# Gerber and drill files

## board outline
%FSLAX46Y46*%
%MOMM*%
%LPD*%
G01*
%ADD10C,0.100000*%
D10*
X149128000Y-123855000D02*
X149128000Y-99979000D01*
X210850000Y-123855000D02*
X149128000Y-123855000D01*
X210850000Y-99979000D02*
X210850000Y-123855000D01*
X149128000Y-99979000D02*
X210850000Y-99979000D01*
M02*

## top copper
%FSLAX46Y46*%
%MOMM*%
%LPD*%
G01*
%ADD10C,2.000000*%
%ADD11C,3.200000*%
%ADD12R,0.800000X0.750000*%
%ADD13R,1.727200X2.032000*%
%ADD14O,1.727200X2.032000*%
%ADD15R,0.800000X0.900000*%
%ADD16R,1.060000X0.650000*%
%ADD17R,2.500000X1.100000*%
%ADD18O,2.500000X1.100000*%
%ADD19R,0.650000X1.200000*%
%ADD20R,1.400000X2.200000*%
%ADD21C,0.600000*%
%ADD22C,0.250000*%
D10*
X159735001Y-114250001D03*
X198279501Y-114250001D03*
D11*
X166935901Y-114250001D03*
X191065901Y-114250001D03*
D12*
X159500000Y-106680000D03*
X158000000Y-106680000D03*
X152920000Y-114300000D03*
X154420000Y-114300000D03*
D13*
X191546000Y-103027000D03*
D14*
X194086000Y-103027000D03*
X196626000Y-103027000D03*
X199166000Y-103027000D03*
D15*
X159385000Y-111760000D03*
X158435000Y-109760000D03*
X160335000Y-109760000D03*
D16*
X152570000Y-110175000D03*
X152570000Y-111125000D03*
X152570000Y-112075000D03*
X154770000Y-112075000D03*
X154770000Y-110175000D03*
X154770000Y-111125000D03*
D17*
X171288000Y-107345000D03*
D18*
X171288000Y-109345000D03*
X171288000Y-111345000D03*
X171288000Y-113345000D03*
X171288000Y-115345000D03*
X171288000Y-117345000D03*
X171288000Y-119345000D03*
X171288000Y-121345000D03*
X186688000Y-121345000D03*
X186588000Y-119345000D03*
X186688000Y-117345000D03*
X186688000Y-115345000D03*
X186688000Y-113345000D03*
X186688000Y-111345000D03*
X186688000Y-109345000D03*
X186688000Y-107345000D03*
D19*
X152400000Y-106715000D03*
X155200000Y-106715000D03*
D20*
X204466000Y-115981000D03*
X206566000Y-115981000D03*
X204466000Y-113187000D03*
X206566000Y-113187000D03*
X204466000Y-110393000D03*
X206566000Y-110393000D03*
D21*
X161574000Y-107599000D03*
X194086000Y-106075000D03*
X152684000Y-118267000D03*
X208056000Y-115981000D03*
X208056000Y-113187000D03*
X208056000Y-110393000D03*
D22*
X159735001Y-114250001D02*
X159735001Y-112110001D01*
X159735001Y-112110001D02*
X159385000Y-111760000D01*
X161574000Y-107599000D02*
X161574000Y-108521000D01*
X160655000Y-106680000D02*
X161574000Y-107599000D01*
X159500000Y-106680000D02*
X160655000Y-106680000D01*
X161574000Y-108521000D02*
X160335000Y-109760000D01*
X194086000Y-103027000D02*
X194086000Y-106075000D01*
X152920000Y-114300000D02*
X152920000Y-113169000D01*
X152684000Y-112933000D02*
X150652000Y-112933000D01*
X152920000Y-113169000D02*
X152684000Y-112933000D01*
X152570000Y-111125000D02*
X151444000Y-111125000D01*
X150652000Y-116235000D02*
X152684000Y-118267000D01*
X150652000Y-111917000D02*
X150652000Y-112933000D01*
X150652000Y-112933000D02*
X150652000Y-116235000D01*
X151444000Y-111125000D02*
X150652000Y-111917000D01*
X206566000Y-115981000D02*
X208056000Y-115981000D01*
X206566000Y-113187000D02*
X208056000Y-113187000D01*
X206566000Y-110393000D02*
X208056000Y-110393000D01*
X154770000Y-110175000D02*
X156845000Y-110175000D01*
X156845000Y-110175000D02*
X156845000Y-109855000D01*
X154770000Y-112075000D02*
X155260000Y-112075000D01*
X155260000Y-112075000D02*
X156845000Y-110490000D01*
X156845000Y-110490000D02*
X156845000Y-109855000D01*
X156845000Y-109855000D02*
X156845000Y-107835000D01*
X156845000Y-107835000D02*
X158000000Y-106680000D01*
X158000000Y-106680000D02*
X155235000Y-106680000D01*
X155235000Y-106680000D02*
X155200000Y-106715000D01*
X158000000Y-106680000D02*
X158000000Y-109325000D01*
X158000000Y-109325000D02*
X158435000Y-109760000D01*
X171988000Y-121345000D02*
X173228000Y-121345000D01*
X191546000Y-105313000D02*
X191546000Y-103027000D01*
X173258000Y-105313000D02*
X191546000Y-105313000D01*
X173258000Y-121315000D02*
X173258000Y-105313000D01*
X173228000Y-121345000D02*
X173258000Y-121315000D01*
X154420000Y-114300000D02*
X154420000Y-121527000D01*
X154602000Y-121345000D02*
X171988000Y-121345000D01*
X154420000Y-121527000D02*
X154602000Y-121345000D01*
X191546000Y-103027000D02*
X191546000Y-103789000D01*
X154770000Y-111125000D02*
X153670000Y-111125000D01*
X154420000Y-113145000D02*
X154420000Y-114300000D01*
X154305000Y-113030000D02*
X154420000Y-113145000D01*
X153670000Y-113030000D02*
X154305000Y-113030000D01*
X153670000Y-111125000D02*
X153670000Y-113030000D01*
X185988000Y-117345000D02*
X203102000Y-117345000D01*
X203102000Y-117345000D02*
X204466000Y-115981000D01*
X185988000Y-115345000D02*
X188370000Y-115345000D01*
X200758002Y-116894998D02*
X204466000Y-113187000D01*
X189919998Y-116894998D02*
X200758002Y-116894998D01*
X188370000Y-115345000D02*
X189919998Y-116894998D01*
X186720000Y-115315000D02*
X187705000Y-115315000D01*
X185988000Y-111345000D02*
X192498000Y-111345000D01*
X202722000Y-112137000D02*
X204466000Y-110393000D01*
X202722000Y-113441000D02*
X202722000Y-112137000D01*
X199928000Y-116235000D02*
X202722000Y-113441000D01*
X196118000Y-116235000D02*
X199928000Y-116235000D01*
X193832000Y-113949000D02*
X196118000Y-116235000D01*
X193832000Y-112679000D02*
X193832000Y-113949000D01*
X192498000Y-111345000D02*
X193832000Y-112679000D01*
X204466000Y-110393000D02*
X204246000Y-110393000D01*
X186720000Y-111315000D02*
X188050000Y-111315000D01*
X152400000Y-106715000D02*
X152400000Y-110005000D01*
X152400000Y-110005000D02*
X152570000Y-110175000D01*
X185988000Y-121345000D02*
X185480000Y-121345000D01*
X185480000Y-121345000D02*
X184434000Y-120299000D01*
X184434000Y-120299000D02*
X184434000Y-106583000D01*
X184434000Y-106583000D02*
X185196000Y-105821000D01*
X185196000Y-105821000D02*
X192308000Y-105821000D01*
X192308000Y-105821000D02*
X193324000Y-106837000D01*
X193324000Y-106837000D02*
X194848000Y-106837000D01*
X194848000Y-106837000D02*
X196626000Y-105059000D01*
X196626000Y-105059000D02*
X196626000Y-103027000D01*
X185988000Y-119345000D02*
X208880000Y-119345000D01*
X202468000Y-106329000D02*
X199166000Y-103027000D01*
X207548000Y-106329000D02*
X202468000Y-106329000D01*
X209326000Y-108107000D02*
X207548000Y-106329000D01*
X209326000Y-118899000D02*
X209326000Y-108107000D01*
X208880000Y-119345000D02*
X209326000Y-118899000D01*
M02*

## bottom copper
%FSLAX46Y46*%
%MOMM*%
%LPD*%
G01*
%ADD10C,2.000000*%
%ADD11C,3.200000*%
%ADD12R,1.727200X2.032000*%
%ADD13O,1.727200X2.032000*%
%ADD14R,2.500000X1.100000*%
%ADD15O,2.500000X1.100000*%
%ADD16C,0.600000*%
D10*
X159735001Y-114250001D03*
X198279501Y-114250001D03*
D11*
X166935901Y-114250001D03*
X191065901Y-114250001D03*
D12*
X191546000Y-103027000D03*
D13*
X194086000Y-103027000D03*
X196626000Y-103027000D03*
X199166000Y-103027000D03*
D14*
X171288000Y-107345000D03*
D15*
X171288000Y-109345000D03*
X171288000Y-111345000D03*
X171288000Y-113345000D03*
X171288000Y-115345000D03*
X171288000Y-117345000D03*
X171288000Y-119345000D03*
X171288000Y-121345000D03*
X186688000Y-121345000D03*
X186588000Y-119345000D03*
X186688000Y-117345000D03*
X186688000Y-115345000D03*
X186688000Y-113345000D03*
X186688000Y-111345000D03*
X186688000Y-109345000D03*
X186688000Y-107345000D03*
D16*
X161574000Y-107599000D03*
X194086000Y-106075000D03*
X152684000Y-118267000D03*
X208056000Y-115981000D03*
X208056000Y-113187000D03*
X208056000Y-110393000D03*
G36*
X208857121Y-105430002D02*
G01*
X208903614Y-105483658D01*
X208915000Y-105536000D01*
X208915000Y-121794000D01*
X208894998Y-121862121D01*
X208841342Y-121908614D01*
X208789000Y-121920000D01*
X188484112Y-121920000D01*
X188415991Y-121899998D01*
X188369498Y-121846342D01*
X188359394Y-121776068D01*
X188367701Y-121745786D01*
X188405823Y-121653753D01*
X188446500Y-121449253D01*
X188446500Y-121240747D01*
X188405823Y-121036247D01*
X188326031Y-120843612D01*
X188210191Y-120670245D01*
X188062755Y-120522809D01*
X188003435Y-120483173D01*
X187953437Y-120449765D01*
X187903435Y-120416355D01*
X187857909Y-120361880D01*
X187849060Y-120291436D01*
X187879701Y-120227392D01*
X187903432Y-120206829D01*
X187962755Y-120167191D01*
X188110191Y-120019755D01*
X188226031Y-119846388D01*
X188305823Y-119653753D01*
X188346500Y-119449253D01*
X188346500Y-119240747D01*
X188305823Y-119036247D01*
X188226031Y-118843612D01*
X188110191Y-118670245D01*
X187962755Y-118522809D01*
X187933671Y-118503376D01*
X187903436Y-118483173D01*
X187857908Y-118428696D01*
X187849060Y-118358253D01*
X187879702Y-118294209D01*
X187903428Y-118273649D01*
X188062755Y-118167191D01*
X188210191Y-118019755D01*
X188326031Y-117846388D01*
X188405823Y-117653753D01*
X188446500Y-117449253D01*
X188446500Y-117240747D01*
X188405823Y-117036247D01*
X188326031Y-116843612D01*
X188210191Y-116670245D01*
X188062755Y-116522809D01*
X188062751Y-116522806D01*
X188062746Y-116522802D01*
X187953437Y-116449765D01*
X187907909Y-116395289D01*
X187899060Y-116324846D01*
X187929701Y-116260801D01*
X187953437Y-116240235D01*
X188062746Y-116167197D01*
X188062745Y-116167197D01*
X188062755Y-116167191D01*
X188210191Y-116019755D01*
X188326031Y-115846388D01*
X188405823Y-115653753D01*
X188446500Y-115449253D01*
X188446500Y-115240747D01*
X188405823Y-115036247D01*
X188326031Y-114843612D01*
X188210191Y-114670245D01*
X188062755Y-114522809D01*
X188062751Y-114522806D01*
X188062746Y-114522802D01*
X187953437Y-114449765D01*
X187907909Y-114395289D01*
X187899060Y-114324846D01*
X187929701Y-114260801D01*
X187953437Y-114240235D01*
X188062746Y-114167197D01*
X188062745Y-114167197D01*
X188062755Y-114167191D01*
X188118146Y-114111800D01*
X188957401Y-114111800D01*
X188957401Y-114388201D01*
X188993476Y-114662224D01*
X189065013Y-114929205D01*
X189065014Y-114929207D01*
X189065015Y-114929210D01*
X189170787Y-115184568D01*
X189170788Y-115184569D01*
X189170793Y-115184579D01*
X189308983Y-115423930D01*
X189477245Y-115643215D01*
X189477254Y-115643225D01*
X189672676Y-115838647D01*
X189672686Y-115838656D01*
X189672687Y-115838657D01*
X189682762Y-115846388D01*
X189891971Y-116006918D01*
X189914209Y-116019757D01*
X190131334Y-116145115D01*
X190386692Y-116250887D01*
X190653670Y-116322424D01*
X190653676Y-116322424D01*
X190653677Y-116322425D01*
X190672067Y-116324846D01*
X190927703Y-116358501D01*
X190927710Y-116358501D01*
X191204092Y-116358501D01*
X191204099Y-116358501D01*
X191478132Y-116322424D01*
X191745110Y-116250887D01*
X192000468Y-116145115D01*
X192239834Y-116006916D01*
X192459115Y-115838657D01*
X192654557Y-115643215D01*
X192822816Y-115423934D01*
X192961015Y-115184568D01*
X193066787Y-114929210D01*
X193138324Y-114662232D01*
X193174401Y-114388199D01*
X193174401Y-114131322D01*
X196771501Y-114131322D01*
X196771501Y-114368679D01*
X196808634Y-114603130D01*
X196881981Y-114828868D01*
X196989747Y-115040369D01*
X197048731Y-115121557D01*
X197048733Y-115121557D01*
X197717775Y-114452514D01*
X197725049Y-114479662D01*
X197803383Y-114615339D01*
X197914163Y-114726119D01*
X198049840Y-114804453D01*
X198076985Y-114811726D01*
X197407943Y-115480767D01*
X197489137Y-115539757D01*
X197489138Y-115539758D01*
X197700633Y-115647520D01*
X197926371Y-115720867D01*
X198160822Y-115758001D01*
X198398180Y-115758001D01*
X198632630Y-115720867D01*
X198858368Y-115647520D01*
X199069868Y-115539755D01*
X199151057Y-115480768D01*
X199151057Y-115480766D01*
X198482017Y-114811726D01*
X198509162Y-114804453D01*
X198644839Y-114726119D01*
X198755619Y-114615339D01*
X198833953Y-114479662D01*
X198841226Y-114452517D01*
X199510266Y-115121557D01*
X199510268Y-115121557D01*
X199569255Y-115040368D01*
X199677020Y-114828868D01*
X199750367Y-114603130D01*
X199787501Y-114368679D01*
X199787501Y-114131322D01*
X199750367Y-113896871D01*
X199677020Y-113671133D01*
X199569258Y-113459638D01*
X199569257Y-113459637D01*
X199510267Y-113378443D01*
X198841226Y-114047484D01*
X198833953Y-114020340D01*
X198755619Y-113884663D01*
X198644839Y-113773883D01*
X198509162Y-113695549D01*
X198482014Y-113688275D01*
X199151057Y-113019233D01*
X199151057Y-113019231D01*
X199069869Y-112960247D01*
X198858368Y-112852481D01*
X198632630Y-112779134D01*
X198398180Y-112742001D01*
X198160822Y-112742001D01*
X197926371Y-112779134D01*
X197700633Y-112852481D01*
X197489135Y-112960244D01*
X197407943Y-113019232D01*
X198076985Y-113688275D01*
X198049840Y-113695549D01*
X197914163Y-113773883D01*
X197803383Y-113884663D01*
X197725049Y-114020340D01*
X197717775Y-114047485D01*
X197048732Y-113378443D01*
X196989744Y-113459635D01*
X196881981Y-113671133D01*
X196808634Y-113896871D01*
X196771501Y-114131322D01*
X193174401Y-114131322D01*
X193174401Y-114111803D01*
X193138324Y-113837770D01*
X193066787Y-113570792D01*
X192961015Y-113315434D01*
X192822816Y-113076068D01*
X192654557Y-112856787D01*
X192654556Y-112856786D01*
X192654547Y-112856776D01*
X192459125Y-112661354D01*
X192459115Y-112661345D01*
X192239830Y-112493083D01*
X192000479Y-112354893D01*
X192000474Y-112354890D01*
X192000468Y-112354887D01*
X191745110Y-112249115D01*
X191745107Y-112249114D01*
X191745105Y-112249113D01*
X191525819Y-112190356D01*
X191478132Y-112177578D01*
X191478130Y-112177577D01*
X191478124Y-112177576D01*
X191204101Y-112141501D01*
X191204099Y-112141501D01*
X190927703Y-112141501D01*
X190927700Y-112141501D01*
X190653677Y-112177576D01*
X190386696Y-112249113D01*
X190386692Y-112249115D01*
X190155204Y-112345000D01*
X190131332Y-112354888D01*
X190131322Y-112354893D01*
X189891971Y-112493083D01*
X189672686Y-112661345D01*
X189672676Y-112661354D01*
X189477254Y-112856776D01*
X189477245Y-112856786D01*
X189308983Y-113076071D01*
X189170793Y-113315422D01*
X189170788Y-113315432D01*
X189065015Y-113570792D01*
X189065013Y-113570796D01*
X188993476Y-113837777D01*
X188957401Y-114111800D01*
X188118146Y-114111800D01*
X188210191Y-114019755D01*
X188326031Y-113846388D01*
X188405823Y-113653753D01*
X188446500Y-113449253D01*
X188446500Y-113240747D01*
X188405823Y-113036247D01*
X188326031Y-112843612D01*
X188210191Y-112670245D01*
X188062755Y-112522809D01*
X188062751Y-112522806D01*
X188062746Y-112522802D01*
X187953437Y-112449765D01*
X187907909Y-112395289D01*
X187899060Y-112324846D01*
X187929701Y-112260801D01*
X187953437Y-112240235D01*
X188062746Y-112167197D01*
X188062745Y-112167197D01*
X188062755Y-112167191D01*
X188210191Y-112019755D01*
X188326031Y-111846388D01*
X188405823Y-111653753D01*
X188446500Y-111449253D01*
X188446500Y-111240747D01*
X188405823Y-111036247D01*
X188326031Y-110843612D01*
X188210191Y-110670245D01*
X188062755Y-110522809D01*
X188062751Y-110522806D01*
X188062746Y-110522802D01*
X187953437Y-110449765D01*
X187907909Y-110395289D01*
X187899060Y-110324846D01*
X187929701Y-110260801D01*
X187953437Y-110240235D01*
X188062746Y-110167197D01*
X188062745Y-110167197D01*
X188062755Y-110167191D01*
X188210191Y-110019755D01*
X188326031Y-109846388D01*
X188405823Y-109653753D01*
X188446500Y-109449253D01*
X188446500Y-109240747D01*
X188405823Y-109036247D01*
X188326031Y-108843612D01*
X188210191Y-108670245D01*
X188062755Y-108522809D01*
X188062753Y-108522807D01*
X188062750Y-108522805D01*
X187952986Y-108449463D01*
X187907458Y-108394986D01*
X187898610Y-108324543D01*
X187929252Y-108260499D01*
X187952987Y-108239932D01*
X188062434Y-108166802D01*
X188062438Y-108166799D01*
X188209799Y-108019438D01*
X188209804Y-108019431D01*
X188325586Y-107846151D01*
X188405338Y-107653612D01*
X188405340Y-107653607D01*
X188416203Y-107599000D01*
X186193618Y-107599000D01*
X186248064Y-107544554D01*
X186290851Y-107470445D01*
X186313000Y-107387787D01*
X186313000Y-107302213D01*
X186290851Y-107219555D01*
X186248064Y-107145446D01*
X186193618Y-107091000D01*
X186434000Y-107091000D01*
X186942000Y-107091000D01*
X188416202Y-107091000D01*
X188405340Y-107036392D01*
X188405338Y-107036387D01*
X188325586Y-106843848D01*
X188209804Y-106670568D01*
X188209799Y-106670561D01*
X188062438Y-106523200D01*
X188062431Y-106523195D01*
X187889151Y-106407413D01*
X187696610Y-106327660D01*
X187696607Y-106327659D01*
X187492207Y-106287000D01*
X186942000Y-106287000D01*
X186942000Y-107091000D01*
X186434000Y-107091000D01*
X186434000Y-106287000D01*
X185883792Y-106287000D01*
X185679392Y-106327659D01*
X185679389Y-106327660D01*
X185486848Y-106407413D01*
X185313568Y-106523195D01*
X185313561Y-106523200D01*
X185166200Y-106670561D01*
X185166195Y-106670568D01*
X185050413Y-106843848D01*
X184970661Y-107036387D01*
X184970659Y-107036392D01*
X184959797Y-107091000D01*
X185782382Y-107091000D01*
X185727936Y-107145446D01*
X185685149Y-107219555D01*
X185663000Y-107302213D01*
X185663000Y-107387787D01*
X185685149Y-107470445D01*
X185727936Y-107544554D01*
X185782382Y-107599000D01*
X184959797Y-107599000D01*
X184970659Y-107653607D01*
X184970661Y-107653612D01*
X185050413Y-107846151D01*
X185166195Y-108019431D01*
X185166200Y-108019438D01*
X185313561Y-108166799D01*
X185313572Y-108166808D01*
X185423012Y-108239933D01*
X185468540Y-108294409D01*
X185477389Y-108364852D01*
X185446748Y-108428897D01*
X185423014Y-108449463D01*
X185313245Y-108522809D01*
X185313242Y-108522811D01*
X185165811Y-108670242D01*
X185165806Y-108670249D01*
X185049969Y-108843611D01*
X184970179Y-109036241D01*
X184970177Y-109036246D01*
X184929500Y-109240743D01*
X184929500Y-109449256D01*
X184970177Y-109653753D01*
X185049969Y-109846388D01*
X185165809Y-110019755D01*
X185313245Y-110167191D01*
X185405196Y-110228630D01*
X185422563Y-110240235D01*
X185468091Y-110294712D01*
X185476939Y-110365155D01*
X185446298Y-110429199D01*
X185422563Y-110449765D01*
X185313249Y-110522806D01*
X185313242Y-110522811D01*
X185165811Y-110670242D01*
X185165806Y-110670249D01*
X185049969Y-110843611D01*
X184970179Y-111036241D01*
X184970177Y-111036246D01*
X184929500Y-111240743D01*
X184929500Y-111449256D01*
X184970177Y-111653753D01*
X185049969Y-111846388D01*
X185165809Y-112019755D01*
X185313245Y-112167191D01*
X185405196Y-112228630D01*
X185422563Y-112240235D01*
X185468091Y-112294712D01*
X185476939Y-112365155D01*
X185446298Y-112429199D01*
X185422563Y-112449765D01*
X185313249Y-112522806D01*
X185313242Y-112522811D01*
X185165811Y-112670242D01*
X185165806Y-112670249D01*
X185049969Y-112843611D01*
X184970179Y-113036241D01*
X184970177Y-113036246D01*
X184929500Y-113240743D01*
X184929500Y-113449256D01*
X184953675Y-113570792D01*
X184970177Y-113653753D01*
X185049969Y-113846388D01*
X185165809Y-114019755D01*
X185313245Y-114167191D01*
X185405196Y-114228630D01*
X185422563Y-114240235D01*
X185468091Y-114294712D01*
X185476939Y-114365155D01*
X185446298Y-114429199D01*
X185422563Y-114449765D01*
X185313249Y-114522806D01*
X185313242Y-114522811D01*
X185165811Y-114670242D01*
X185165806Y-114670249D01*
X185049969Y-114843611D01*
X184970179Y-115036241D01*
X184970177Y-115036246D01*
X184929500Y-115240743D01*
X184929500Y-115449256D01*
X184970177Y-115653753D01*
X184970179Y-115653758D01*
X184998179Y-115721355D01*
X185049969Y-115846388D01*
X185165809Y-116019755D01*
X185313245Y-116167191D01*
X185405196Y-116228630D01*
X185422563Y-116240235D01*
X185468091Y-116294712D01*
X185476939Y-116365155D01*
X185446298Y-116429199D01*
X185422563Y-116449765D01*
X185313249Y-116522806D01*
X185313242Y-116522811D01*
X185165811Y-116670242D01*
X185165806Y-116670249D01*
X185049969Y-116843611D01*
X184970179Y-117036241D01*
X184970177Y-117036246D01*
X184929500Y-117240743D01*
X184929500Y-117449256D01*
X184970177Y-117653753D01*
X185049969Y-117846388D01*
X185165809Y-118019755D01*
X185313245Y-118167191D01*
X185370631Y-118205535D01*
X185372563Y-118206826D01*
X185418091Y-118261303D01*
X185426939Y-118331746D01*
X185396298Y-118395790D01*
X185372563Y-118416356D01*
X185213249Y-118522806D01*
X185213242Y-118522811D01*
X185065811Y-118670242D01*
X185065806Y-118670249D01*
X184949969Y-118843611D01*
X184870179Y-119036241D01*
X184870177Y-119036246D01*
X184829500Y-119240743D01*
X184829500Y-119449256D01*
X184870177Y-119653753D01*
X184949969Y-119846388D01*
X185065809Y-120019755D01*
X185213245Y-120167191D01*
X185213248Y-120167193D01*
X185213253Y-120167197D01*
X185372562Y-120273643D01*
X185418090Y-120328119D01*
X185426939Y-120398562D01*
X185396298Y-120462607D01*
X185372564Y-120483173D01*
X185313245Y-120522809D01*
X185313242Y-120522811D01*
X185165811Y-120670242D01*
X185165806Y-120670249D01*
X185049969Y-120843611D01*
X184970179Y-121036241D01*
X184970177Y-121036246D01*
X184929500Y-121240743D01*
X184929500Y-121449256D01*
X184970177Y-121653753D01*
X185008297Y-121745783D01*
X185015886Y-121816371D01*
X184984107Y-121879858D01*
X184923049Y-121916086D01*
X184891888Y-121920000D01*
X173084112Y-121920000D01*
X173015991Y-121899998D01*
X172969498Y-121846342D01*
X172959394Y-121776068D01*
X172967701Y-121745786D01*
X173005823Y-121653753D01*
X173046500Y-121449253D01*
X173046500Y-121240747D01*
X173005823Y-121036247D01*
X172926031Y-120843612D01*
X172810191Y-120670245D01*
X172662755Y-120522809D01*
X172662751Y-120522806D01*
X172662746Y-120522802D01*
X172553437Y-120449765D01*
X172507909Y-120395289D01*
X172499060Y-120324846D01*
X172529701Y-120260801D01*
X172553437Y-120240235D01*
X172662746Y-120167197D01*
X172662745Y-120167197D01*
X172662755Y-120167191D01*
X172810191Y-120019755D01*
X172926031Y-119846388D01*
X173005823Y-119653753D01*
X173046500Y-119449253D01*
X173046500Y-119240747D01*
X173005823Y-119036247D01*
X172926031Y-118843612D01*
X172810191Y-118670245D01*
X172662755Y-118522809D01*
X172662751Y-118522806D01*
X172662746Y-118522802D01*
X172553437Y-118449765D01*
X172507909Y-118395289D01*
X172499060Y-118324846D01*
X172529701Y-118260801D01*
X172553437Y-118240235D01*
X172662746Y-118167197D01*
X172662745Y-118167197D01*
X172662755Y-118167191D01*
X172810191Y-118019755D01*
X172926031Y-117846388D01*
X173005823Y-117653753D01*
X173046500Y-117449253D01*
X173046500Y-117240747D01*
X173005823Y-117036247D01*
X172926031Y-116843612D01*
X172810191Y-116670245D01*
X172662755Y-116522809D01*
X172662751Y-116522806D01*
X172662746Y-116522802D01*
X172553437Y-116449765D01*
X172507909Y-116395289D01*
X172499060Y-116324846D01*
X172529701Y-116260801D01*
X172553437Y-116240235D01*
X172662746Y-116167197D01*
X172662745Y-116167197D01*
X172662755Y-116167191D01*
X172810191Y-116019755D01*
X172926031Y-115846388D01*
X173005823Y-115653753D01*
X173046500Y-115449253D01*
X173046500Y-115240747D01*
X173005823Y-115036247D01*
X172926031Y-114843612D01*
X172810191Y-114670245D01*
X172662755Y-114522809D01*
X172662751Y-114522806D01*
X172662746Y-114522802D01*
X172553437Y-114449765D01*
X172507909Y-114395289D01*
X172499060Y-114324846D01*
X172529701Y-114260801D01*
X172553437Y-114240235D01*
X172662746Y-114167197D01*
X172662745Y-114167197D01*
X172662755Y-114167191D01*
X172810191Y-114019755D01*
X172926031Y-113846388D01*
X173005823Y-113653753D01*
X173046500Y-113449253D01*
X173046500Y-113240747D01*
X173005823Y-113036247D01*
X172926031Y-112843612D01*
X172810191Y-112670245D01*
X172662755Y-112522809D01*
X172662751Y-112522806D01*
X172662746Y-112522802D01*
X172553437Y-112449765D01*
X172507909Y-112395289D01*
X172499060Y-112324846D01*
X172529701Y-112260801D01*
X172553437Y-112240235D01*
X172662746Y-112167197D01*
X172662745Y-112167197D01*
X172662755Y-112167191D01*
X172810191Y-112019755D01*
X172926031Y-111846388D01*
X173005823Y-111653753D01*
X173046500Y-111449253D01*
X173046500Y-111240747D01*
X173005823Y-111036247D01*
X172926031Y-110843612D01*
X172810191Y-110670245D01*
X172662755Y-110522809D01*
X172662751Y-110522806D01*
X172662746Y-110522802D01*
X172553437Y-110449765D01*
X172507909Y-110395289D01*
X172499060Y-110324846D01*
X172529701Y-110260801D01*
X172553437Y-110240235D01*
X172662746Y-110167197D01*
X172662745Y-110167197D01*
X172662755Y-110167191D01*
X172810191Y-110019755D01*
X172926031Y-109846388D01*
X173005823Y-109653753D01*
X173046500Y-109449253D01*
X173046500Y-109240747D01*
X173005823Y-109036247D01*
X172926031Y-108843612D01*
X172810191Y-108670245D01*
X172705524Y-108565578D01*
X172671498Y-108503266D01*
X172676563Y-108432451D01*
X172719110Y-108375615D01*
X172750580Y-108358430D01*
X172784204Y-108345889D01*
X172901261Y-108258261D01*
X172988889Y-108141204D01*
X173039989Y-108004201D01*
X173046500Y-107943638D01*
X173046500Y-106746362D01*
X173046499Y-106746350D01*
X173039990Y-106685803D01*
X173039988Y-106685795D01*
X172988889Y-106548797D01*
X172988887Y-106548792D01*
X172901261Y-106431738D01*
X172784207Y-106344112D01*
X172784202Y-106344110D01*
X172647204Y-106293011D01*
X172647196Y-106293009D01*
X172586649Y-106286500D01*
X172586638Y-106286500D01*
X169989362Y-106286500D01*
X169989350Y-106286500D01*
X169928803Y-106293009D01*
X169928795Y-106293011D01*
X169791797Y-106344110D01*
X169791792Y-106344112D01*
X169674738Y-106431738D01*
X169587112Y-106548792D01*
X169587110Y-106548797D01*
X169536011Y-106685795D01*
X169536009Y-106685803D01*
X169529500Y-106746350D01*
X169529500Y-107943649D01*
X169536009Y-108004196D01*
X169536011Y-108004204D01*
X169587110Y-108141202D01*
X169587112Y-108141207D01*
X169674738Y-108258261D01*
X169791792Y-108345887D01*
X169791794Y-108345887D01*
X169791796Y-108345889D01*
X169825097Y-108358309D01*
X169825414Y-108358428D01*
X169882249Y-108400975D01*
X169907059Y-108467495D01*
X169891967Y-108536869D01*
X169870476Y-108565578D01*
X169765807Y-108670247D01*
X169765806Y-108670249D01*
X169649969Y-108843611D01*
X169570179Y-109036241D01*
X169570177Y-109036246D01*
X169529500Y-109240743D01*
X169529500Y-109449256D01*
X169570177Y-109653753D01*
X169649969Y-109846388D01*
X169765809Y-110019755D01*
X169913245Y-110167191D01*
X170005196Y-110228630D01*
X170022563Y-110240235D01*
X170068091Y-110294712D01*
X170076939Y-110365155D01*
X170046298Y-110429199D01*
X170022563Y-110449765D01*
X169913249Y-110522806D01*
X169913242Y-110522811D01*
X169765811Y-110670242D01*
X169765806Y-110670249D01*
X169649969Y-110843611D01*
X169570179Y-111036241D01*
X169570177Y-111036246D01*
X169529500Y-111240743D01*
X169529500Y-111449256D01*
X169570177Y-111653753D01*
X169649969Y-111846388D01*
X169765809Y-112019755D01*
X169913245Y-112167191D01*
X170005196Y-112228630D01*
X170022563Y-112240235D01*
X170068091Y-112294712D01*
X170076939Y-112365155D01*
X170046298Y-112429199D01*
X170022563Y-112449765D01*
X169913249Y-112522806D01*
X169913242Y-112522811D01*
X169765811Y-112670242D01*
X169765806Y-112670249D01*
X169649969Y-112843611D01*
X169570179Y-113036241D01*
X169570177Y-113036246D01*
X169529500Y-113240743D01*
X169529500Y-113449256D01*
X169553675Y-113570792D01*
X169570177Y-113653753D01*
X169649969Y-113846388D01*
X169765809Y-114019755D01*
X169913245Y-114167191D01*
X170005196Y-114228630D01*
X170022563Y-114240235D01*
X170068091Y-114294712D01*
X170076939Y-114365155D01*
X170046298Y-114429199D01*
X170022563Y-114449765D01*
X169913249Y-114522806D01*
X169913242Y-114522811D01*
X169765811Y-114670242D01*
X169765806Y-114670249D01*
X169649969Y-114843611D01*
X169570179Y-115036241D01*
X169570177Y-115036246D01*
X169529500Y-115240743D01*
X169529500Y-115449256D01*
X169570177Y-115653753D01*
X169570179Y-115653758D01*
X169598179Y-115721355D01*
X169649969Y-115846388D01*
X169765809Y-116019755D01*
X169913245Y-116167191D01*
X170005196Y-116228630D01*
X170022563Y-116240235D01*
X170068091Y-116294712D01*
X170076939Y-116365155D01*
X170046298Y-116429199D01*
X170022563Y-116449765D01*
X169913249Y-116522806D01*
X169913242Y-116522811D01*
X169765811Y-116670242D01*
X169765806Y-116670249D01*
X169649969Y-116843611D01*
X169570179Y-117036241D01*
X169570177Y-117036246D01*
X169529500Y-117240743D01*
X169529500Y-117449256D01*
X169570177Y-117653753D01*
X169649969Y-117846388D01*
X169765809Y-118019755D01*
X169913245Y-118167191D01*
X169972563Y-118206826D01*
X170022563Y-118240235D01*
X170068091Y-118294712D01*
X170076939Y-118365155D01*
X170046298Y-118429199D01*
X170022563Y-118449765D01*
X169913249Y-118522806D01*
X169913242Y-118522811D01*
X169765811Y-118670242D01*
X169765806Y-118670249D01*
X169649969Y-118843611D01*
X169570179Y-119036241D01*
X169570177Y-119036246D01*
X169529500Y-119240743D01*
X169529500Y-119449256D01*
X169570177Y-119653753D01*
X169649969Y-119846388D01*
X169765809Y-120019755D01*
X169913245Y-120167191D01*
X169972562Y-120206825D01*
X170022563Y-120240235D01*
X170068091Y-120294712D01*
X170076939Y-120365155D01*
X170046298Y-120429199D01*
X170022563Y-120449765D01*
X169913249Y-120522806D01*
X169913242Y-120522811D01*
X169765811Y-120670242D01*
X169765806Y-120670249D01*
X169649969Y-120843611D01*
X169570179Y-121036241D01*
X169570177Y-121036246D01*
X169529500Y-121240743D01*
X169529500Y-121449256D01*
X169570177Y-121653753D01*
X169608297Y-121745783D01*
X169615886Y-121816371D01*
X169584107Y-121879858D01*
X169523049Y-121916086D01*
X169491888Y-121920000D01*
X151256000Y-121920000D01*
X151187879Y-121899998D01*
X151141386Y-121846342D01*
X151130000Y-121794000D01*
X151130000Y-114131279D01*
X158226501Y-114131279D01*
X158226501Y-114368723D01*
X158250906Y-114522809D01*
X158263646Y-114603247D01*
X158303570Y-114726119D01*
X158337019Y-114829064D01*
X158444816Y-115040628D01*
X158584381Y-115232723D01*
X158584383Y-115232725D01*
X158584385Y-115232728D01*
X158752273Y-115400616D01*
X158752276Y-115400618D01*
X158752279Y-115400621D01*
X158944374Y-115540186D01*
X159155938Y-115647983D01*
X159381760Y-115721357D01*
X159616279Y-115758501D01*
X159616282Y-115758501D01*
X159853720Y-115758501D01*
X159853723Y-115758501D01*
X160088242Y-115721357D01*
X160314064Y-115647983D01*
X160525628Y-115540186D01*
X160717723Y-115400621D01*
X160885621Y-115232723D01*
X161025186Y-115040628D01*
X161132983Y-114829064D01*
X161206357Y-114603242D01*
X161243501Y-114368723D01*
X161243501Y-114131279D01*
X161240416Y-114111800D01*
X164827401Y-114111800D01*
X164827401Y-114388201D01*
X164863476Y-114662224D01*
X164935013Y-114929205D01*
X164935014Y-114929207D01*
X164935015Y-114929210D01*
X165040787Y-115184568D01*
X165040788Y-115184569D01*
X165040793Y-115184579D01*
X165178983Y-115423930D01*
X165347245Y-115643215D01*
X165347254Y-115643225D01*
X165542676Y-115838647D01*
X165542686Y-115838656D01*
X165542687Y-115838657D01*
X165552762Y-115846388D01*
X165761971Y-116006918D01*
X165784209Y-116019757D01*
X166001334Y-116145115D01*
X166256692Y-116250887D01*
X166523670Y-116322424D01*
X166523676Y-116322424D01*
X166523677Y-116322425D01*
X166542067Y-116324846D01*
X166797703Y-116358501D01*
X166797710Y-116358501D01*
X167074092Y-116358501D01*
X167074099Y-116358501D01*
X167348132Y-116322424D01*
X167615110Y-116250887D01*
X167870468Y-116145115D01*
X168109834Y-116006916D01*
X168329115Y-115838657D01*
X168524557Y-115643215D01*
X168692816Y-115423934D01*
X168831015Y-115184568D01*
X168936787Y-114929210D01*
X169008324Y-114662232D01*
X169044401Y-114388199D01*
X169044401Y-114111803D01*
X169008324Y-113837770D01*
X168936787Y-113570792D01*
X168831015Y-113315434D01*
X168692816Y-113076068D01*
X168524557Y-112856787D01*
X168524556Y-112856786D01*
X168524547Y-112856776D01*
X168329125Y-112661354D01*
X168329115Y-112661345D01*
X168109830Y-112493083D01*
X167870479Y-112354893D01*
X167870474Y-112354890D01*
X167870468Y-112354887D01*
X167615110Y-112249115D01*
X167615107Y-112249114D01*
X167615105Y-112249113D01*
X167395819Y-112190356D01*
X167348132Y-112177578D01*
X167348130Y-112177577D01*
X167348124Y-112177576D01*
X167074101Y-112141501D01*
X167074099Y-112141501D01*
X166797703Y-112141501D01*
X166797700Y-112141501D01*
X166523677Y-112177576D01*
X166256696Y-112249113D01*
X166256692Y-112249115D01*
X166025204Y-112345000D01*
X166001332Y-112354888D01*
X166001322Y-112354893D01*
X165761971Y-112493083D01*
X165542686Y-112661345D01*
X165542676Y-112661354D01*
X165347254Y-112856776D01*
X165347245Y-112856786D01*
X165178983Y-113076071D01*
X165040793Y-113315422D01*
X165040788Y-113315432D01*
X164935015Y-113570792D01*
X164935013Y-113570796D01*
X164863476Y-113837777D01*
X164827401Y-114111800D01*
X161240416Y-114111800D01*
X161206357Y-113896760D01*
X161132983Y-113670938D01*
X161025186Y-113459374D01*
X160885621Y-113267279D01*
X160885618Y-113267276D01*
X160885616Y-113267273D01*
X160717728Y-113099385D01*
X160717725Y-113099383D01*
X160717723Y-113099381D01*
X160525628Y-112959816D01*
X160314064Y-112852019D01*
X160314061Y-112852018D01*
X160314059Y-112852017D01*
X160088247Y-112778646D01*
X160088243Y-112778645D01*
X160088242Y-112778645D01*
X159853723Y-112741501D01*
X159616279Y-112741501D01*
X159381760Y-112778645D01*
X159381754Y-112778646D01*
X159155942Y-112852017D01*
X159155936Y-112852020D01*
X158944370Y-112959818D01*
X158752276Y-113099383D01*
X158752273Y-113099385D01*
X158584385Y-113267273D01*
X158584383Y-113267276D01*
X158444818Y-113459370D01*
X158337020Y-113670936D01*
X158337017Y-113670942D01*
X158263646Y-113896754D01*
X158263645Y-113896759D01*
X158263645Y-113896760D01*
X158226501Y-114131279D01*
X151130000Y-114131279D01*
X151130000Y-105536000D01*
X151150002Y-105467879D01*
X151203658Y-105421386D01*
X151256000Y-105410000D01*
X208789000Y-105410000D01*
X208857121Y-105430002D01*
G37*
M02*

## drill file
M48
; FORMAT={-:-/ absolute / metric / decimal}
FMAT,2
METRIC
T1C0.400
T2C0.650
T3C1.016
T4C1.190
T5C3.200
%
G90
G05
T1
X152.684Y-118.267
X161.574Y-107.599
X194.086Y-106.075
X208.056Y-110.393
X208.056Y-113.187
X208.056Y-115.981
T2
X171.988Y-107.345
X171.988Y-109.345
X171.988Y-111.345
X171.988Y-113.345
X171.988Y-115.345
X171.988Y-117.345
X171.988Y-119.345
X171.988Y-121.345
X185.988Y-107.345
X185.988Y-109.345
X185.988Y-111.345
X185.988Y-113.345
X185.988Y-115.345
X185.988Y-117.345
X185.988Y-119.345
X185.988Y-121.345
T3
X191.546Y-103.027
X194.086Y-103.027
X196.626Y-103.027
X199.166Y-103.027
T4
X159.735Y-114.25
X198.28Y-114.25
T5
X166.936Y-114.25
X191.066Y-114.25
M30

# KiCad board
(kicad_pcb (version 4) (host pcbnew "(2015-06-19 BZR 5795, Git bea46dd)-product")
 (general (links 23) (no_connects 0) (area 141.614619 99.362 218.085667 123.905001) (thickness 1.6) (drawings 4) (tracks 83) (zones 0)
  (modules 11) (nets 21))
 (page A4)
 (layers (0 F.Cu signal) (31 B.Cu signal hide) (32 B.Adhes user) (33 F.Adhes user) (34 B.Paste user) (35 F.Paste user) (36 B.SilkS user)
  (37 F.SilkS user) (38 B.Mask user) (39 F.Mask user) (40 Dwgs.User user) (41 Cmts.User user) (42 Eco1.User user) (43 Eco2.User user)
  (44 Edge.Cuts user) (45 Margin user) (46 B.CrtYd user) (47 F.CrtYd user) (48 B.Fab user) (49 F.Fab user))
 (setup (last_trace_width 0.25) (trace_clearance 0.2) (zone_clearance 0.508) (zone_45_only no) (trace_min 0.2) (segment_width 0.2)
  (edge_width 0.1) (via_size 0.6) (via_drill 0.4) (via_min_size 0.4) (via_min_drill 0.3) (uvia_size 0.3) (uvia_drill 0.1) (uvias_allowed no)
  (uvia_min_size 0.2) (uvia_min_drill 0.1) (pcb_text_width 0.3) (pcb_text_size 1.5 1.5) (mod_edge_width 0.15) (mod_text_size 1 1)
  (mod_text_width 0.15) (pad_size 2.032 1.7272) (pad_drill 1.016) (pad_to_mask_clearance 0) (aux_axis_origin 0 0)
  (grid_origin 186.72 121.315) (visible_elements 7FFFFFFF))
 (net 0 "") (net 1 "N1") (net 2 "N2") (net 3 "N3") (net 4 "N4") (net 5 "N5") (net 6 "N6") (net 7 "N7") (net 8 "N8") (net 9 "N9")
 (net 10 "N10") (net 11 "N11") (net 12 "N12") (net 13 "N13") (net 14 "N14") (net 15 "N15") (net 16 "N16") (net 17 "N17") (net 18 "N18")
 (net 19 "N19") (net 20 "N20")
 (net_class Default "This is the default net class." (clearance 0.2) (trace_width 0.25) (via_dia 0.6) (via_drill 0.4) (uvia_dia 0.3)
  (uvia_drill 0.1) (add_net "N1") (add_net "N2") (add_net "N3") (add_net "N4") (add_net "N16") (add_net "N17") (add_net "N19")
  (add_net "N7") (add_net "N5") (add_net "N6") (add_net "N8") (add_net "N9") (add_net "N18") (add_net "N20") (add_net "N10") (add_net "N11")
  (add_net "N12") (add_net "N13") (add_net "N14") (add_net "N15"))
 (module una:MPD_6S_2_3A (layer B.Cu) (at 159.735001 114.250001)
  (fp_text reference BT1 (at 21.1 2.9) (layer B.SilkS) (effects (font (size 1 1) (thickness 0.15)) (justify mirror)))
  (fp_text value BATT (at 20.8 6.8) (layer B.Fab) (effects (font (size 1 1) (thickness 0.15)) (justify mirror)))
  (pad 1 thru_hole circle (at 0 0) (size 2 2) (drill 1.19) (layers *.Cu *.Mask B.SilkS) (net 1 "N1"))
  (pad 2 thru_hole circle (at 38.5445 0) (size 2 2) (drill 1.19) (layers *.Cu *.Mask B.SilkS) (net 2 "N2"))
  (pad "" thru_hole circle (at 7.2009 0) (size 3.2 3.2) (drill 3.2) (layers *.Cu *.Mask B.SilkS))
  (pad "" thru_hole circle (at 31.3309 0) (size 3.2 3.2) (drill 3.2) (layers *.Cu *.Mask B.SilkS)))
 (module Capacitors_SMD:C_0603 (layer F.Cu) (at 158.75 106.68 180)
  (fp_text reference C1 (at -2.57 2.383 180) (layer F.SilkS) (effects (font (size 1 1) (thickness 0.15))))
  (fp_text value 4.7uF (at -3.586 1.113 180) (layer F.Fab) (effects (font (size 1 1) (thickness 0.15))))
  (pad 1 smd rect (at -0.75 0 180) (size 0.8 0.75) (layers F.Cu F.Paste F.Mask) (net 2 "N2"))
  (pad 2 smd rect (at 0.75 0 180) (size 0.8 0.75) (layers F.Cu F.Paste F.Mask) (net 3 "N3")))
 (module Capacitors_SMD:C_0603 (layer F.Cu) (at 153.67 114.3)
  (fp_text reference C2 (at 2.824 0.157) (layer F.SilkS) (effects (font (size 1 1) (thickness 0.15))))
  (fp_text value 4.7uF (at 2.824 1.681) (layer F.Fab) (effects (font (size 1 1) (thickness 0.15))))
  (pad 1 smd rect (at -0.75 0) (size 0.8 0.75) (layers F.Cu F.Paste F.Mask) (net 2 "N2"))
  (pad 2 smd rect (at 0.75 0) (size 0.8 0.75) (layers F.Cu F.Paste F.Mask) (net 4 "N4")))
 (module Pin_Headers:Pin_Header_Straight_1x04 (layer F.Cu) (at 191.546 103.027 90)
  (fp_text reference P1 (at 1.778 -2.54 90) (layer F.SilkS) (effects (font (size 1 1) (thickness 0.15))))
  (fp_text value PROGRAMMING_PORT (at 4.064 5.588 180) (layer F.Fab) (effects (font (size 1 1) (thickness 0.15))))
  (pad 1 thru_hole rect (at 0 0 90) (size 2.032 1.7272) (drill 1.016) (layers *.Cu *.Mask F.SilkS) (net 4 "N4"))
  (pad 2 thru_hole oval (at 0 2.54 90) (size 2.032 1.7272) (drill 1.016) (layers *.Cu *.Mask F.SilkS) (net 2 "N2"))
  (pad 3 thru_hole oval (at 0 5.08 90) (size 2.032 1.7272) (drill 1.016) (layers *.Cu *.Mask F.SilkS) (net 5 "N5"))
  (pad 4 thru_hole oval (at 0 7.62 90) (size 2.032 1.7272) (drill 1.016) (layers *.Cu *.Mask F.SilkS) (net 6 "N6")))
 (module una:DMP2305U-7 (layer F.Cu) (at 159.385 111.76 180)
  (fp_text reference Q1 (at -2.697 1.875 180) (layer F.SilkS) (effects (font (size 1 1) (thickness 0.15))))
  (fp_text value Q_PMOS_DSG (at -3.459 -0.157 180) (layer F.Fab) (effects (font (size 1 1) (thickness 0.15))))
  (pad 1 smd rect (at 0 0 180) (size 0.8 0.9) (layers F.Cu F.Paste F.Mask) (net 1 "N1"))
  (pad 2 smd rect (at 0.95 2 180) (size 0.8 0.9) (layers F.Cu F.Paste F.Mask) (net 3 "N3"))
  (pad 3 smd rect (at -0.95 2 180) (size 0.8 0.9) (layers F.Cu F.Paste F.Mask) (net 2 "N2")))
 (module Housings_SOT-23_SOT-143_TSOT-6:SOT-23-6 (layer F.Cu) (at 153.67 111.125)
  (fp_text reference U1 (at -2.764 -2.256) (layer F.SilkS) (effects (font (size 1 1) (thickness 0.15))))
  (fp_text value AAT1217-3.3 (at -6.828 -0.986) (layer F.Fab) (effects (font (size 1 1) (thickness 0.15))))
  (pad 1 smd rect (at -1.1 -0.95) (size 1.06 0.65) (layers F.Cu F.Paste F.Mask) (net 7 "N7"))
  (pad 2 smd rect (at -1.1 0) (size 1.06 0.65) (layers F.Cu F.Paste F.Mask) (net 2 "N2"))
  (pad 3 smd rect (at -1.1 0.95) (size 1.06 0.65) (layers F.Cu F.Paste F.Mask) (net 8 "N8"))
  (pad 4 smd rect (at 1.1 0.95) (size 1.06 0.65) (layers F.Cu F.Paste F.Mask) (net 3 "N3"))
  (pad 6 smd rect (at 1.1 -0.95) (size 1.06 0.65) (layers F.Cu F.Paste F.Mask) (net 3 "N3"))
  (pad 5 smd rect (at 1.1 0) (size 1.06 0.65) (layers F.Cu F.Paste F.Mask) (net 4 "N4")))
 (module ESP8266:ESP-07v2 (layer F.Cu) (at 171.988 107.345)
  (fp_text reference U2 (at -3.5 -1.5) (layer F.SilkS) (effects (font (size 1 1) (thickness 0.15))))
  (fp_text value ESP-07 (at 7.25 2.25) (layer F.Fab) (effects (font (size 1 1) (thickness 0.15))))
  (pad 1 thru_hole rect (at 0 0) (size 2.5 1.1) (drill 0.65 (offset -0.7 0)) (layers *.Cu *.Mask F.SilkS) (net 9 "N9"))
  (pad 2 thru_hole oval (at 0 2) (size 2.5 1.1) (drill 0.65 (offset -0.7 0)) (layers *.Cu *.Mask F.SilkS) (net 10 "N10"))
  (pad 3 thru_hole oval (at 0 4) (size 2.5 1.1) (drill 0.65 (offset -0.7 0)) (layers *.Cu *.Mask F.SilkS) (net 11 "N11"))
  (pad 4 thru_hole oval (at 0 6) (size 2.5 1.1) (drill 0.65 (offset -0.7 0)) (layers *.Cu *.Mask F.SilkS) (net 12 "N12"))
  (pad 5 thru_hole oval (at 0 8) (size 2.5 1.1) (drill 0.65 (offset -0.7 0)) (layers *.Cu *.Mask F.SilkS) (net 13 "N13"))
  (pad 6 thru_hole oval (at 0 10) (size 2.5 1.1) (drill 0.65 (offset -0.7 0)) (layers *.Cu *.Mask F.SilkS) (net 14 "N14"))
  (pad 7 thru_hole oval (at 0 12) (size 2.5 1.1) (drill 0.65 (offset -0.7 0)) (layers *.Cu *.Mask F.SilkS) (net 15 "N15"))
  (pad 8 thru_hole oval (at 0 14) (size 2.5 1.1) (drill 0.65 (offset -0.7 0)) (layers *.Cu *.Mask F.SilkS) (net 4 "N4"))
  (pad 9 thru_hole oval (at 14 14) (size 2.5 1.1) (drill 0.65 (offset 0.7 0)) (layers *.Cu *.Mask F.SilkS) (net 5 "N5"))
  (pad 10 thru_hole oval (at 14 12) (size 2.5 1.1) (drill 0.65 (offset 0.6 0)) (layers *.Cu *.Mask F.SilkS) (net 6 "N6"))
  (pad 11 thru_hole oval (at 14 10) (size 2.5 1.1) (drill 0.65 (offset 0.7 0)) (layers *.Cu *.Mask F.SilkS) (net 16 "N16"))
  (pad 12 thru_hole oval (at 14 8) (size 2.5 1.1) (drill 0.65 (offset 0.7 0)) (layers *.Cu *.Mask F.SilkS) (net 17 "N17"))
  (pad 13 thru_hole oval (at 14 6) (size 2.5 1.1) (drill 0.65 (offset 0.7 0)) (layers *.Cu *.Mask F.SilkS) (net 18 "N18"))
  (pad 14 thru_hole oval (at 14 4) (size 2.5 1.1) (drill 0.65 (offset 0.7 0)) (layers *.Cu *.Mask F.SilkS) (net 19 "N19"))
  (pad 15 thru_hole oval (at 14 2) (size 2.5 1.1) (drill 0.65 (offset 0.7 0)) (layers *.Cu *.Mask F.SilkS) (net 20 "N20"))
  (pad 16 thru_hole oval (at 14 0) (size 2.5 1.1) (drill 0.65 (offset 0.7 0)) (layers *.Cu *.Mask F.SilkS) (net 2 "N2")))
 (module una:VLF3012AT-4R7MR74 (layer F.Cu) (at 152.4 107.315)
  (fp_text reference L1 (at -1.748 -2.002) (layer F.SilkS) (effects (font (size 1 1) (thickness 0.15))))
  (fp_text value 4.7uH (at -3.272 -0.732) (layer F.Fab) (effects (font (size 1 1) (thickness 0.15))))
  (pad 1 smd rect (at 0 -0.6) (size 0.65 1.2) (layers F.Cu F.Paste F.Mask) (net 7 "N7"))
  (pad 2 smd rect (at 2.8 -0.6) (size 0.65 1.2) (layers F.Cu F.Paste F.Mask) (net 3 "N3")))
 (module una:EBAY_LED (layer F.Cu) (at 205.516 115.981)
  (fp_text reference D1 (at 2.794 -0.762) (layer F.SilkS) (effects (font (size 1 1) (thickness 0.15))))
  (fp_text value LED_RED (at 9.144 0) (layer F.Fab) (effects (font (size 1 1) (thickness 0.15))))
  (pad 2 smd rect (at -1.05 0) (size 1.4 2.2) (layers F.Cu F.Paste F.Mask) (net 16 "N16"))
  (pad 1 smd rect (at 1.05 0) (size 1.4 2.2) (layers F.Cu F.Paste F.Mask) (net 2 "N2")))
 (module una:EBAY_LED (layer F.Cu) (at 205.516 113.187)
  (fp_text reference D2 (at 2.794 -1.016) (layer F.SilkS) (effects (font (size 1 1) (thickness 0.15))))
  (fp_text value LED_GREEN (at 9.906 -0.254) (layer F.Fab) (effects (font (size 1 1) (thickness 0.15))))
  (pad 2 smd rect (at -1.05 0) (size 1.4 2.2) (layers F.Cu F.Paste F.Mask) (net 17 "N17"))
  (pad 1 smd rect (at 1.05 0) (size 1.4 2.2) (layers F.Cu F.Paste F.Mask) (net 2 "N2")))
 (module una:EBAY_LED (layer F.Cu) (at 205.516 110.393)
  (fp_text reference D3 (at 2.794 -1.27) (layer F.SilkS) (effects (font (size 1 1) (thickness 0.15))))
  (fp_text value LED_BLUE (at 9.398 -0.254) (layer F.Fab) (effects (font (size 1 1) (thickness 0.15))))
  (pad 2 smd rect (at -1.05 0) (size 1.4 2.2) (layers F.Cu F.Paste F.Mask) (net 19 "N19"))
  (pad 1 smd rect (at 1.05 0) (size 1.4 2.2) (layers F.Cu F.Paste F.Mask) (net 2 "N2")))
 (gr_line (start 149.128 123.855) (end 149.128 99.979) (angle 90) (layer Edge.Cuts) (width 0.1))
 (gr_line (start 210.85 123.855) (end 149.128 123.855) (angle 90) (layer Edge.Cuts) (width 0.1))
 (gr_line (start 210.85 99.979) (end 210.85 123.855) (angle 90) (layer Edge.Cuts) (width 0.1))
 (gr_line (start 149.128 99.979) (end 210.85 99.979) (angle 90) (layer Edge.Cuts) (width 0.1))
 (segment (start 159.735001 114.250001) (end 159.735001 112.110001) (width 0.25) (layer F.Cu) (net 1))
 (segment (start 159.735001 112.110001) (end 159.385 111.76) (width 0.25) (layer F.Cu) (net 1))
 (segment (start 161.574 107.599) (end 161.574 108.521) (width 0.25) (layer F.Cu) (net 2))
 (segment (start 160.655 106.68) (end 161.574 107.599) (width 0.25) (layer F.Cu) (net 2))
 (via (at 161.574 107.599) (size 0.6) (drill 0.4) (layers F.Cu B.Cu) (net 2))
 (segment (start 159.5 106.68) (end 160.655 106.68) (width 0.25) (layer F.Cu) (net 2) (status 400000))
 (segment (start 161.574 108.521) (end 160.335 109.76) (width 0.25) (layer F.Cu) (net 2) (status 800000))
 (segment (start 194.086 103.027) (end 194.086 106.075) (width 0.25) (layer F.Cu) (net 2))
 (via (at 194.086 106.075) (size 0.6) (drill 0.4) (layers F.Cu B.Cu) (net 2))
 (segment (start 152.92 114.3) (end 152.92 113.169) (width 0.25) (layer F.Cu) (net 2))
 (segment (start 152.684 112.933) (end 150.652 112.933) (width 0.25) (layer F.Cu) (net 2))
 (segment (start 152.92 113.169) (end 152.684 112.933) (width 0.25) (layer F.Cu) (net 2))
 (segment (start 152.57 111.125) (end 151.444 111.125) (width 0.25) (layer F.Cu) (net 2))
 (via (at 152.684 118.267) (size 0.6) (drill 0.4) (layers F.Cu B.Cu) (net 2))
 (segment (start 150.652 116.235) (end 152.684 118.267) (width 0.25) (layer F.Cu) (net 2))
 (segment (start 150.652 111.917) (end 150.652 112.933) (width 0.25) (layer F.Cu) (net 2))
 (segment (start 150.652 112.933) (end 150.652 116.235) (width 0.25) (layer F.Cu) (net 2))
 (segment (start 151.444 111.125) (end 150.652 111.917) (width 0.25) (layer F.Cu) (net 2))
 (segment (start 206.566 115.981) (end 208.056 115.981) (width 0.25) (layer F.Cu) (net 2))
 (via (at 208.056 115.981) (size 0.6) (drill 0.4) (layers F.Cu B.Cu) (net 2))
 (segment (start 206.566 113.187) (end 208.056 113.187) (width 0.25) (layer F.Cu) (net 2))
 (via (at 208.056 113.187) (size 0.6) (drill 0.4) (layers F.Cu B.Cu) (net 2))
 (segment (start 206.566 110.393) (end 208.056 110.393) (width 0.25) (layer F.Cu) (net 2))
 (via (at 208.056 110.393) (size 0.6) (drill 0.4) (layers F.Cu B.Cu) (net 2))
 (segment (start 154.77 110.175) (end 156.845 110.175) (width 0.25) (layer F.Cu) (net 3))
 (segment (start 156.845 110.175) (end 156.845 109.855) (width 0.25) (layer F.Cu) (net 3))
 (segment (start 154.77 112.075) (end 155.26 112.075) (width 0.25) (layer F.Cu) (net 3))
 (segment (start 155.26 112.075) (end 156.845 110.49) (width 0.25) (layer F.Cu) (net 3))
 (segment (start 156.845 110.49) (end 156.845 109.855) (width 0.25) (layer F.Cu) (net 3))
 (segment (start 156.845 109.855) (end 156.845 107.835) (width 0.25) (layer F.Cu) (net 3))
 (segment (start 156.845 107.835) (end 158 106.68) (width 0.25) (layer F.Cu) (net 3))
 (segment (start 158 106.68) (end 155.235 106.68) (width 0.25) (layer F.Cu) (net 3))
 (segment (start 155.235 106.68) (end 155.2 106.715) (width 0.25) (layer F.Cu) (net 3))
 (segment (start 158 106.68) (end 158 109.325) (width 0.25) (layer F.Cu) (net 3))
 (segment (start 158 109.325) (end 158.435 109.76) (width 0.25) (layer F.Cu) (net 3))
 (segment (start 171.988 121.345) (end 173.228 121.345) (width 0.25) (layer F.Cu) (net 4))
 (segment (start 191.546 105.313) (end 191.546 103.027) (width 0.25) (layer F.Cu) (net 4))
 (segment (start 173.258 105.313) (end 191.546 105.313) (width 0.25) (layer F.Cu) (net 4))
 (segment (start 173.258 121.315) (end 173.258 105.313) (width 0.25) (layer F.Cu) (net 4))
 (segment (start 173.228 121.345) (end 173.258 121.315) (width 0.25) (layer F.Cu) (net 4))
 (segment (start 154.42 114.3) (end 154.42 121.527) (width 0.25) (layer F.Cu) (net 4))
 (segment (start 154.602 121.345) (end 171.988 121.345) (width 0.25) (layer F.Cu) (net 4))
 (segment (start 154.42 121.527) (end 154.602 121.345) (width 0.25) (layer F.Cu) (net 4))
 (segment (start 191.546 103.027) (end 191.546 103.789) (width 0.25) (layer F.Cu) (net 4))
 (segment (start 154.77 111.125) (end 153.67 111.125) (width 0.25) (layer F.Cu) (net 4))
 (segment (start 154.42 113.145) (end 154.42 114.3) (width 0.25) (layer F.Cu) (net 4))
 (segment (start 154.305 113.03) (end 154.42 113.145) (width 0.25) (layer F.Cu) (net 4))
 (segment (start 153.67 113.03) (end 154.305 113.03) (width 0.25) (layer F.Cu) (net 4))
 (segment (start 153.67 111.125) (end 153.67 113.03) (width 0.25) (layer F.Cu) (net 4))
 (segment (start 185.988 117.345) (end 203.102 117.345) (width 0.25) (layer F.Cu) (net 16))
 (segment (start 203.102 117.345) (end 204.466 115.981) (width 0.25) (layer F.Cu) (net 16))
 (segment (start 185.988 115.345) (end 188.37 115.345) (width 0.25) (layer F.Cu) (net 17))
 (segment (start 200.758002 116.894998) (end 204.466 113.187) (width 0.25) (layer F.Cu) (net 17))
 (segment (start 189.919998 116.894998) (end 200.758002 116.894998) (width 0.25) (layer F.Cu) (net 17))
 (segment (start 188.37 115.345) (end 189.919998 116.894998) (width 0.25) (layer F.Cu) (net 17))
 (segment (start 186.72 115.315) (end 187.705 115.315) (width 0.25) (layer F.Cu) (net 17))
 (segment (start 185.988 111.345) (end 192.498 111.345) (width 0.25) (layer F.Cu) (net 19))
 (segment (start 202.722 112.137) (end 204.466 110.393) (width 0.25) (layer F.Cu) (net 19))
 (segment (start 202.722 113.441) (end 202.722 112.137) (width 0.25) (layer F.Cu) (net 19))
 (segment (start 199.928 116.235) (end 202.722 113.441) (width 0.25) (layer F.Cu) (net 19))
 (segment (start 196.118 116.235) (end 199.928 116.235) (width 0.25) (layer F.Cu) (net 19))
 (segment (start 193.832 113.949) (end 196.118 116.235) (width 0.25) (layer F.Cu) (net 19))
 (segment (start 193.832 112.679) (end 193.832 113.949) (width 0.25) (layer F.Cu) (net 19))
 (segment (start 192.498 111.345) (end 193.832 112.679) (width 0.25) (layer F.Cu) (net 19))
 (segment (start 204.466 110.393) (end 204.246 110.393) (width 0.25) (layer F.Cu) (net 19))
 (segment (start 186.72 111.315) (end 188.05 111.315) (width 0.25) (layer F.Cu) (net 19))
 (segment (start 152.4 106.715) (end 152.4 110.005) (width 0.25) (layer F.Cu) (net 7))
 (segment (start 152.4 110.005) (end 152.57 110.175) (width 0.25) (layer F.Cu) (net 7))
 (segment (start 185.988 121.345) (end 185.48 121.345) (width 0.25) (layer F.Cu) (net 5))
 (segment (start 185.48 121.345) (end 184.434 120.299) (width 0.25) (layer F.Cu) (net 5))
 (segment (start 184.434 120.299) (end 184.434 106.583) (width 0.25) (layer F.Cu) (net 5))
 (segment (start 184.434 106.583) (end 185.196 105.821) (width 0.25) (layer F.Cu) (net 5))
 (segment (start 185.196 105.821) (end 192.308 105.821) (width 0.25) (layer F.Cu) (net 5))
 (segment (start 192.308 105.821) (end 193.324 106.837) (width 0.25) (layer F.Cu) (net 5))
 (segment (start 193.324 106.837) (end 194.848 106.837) (width 0.25) (layer F.Cu) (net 5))
 (segment (start 194.848 106.837) (end 196.626 105.059) (width 0.25) (layer F.Cu) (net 5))
 (segment (start 196.626 105.059) (end 196.626 103.027) (width 0.25) (layer F.Cu) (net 5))
 (segment (start 185.988 119.345) (end 208.88 119.345) (width 0.25) (layer F.Cu) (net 6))
 (segment (start 202.468 106.329) (end 199.166 103.027) (width 0.25) (layer F.Cu) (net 6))
 (segment (start 207.548 106.329) (end 202.468 106.329) (width 0.25) (layer F.Cu) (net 6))
 (segment (start 209.326 108.107) (end 207.548 106.329) (width 0.25) (layer F.Cu) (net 6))
 (segment (start 209.326 118.899) (end 209.326 108.107) (width 0.25) (layer F.Cu) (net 6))
 (segment (start 208.88 119.345) (end 209.326 118.899) (width 0.25) (layer F.Cu) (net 6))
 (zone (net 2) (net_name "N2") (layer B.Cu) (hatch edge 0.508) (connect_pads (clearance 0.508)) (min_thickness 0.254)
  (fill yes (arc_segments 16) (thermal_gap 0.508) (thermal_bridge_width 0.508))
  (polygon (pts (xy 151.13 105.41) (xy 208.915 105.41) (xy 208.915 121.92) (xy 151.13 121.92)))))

